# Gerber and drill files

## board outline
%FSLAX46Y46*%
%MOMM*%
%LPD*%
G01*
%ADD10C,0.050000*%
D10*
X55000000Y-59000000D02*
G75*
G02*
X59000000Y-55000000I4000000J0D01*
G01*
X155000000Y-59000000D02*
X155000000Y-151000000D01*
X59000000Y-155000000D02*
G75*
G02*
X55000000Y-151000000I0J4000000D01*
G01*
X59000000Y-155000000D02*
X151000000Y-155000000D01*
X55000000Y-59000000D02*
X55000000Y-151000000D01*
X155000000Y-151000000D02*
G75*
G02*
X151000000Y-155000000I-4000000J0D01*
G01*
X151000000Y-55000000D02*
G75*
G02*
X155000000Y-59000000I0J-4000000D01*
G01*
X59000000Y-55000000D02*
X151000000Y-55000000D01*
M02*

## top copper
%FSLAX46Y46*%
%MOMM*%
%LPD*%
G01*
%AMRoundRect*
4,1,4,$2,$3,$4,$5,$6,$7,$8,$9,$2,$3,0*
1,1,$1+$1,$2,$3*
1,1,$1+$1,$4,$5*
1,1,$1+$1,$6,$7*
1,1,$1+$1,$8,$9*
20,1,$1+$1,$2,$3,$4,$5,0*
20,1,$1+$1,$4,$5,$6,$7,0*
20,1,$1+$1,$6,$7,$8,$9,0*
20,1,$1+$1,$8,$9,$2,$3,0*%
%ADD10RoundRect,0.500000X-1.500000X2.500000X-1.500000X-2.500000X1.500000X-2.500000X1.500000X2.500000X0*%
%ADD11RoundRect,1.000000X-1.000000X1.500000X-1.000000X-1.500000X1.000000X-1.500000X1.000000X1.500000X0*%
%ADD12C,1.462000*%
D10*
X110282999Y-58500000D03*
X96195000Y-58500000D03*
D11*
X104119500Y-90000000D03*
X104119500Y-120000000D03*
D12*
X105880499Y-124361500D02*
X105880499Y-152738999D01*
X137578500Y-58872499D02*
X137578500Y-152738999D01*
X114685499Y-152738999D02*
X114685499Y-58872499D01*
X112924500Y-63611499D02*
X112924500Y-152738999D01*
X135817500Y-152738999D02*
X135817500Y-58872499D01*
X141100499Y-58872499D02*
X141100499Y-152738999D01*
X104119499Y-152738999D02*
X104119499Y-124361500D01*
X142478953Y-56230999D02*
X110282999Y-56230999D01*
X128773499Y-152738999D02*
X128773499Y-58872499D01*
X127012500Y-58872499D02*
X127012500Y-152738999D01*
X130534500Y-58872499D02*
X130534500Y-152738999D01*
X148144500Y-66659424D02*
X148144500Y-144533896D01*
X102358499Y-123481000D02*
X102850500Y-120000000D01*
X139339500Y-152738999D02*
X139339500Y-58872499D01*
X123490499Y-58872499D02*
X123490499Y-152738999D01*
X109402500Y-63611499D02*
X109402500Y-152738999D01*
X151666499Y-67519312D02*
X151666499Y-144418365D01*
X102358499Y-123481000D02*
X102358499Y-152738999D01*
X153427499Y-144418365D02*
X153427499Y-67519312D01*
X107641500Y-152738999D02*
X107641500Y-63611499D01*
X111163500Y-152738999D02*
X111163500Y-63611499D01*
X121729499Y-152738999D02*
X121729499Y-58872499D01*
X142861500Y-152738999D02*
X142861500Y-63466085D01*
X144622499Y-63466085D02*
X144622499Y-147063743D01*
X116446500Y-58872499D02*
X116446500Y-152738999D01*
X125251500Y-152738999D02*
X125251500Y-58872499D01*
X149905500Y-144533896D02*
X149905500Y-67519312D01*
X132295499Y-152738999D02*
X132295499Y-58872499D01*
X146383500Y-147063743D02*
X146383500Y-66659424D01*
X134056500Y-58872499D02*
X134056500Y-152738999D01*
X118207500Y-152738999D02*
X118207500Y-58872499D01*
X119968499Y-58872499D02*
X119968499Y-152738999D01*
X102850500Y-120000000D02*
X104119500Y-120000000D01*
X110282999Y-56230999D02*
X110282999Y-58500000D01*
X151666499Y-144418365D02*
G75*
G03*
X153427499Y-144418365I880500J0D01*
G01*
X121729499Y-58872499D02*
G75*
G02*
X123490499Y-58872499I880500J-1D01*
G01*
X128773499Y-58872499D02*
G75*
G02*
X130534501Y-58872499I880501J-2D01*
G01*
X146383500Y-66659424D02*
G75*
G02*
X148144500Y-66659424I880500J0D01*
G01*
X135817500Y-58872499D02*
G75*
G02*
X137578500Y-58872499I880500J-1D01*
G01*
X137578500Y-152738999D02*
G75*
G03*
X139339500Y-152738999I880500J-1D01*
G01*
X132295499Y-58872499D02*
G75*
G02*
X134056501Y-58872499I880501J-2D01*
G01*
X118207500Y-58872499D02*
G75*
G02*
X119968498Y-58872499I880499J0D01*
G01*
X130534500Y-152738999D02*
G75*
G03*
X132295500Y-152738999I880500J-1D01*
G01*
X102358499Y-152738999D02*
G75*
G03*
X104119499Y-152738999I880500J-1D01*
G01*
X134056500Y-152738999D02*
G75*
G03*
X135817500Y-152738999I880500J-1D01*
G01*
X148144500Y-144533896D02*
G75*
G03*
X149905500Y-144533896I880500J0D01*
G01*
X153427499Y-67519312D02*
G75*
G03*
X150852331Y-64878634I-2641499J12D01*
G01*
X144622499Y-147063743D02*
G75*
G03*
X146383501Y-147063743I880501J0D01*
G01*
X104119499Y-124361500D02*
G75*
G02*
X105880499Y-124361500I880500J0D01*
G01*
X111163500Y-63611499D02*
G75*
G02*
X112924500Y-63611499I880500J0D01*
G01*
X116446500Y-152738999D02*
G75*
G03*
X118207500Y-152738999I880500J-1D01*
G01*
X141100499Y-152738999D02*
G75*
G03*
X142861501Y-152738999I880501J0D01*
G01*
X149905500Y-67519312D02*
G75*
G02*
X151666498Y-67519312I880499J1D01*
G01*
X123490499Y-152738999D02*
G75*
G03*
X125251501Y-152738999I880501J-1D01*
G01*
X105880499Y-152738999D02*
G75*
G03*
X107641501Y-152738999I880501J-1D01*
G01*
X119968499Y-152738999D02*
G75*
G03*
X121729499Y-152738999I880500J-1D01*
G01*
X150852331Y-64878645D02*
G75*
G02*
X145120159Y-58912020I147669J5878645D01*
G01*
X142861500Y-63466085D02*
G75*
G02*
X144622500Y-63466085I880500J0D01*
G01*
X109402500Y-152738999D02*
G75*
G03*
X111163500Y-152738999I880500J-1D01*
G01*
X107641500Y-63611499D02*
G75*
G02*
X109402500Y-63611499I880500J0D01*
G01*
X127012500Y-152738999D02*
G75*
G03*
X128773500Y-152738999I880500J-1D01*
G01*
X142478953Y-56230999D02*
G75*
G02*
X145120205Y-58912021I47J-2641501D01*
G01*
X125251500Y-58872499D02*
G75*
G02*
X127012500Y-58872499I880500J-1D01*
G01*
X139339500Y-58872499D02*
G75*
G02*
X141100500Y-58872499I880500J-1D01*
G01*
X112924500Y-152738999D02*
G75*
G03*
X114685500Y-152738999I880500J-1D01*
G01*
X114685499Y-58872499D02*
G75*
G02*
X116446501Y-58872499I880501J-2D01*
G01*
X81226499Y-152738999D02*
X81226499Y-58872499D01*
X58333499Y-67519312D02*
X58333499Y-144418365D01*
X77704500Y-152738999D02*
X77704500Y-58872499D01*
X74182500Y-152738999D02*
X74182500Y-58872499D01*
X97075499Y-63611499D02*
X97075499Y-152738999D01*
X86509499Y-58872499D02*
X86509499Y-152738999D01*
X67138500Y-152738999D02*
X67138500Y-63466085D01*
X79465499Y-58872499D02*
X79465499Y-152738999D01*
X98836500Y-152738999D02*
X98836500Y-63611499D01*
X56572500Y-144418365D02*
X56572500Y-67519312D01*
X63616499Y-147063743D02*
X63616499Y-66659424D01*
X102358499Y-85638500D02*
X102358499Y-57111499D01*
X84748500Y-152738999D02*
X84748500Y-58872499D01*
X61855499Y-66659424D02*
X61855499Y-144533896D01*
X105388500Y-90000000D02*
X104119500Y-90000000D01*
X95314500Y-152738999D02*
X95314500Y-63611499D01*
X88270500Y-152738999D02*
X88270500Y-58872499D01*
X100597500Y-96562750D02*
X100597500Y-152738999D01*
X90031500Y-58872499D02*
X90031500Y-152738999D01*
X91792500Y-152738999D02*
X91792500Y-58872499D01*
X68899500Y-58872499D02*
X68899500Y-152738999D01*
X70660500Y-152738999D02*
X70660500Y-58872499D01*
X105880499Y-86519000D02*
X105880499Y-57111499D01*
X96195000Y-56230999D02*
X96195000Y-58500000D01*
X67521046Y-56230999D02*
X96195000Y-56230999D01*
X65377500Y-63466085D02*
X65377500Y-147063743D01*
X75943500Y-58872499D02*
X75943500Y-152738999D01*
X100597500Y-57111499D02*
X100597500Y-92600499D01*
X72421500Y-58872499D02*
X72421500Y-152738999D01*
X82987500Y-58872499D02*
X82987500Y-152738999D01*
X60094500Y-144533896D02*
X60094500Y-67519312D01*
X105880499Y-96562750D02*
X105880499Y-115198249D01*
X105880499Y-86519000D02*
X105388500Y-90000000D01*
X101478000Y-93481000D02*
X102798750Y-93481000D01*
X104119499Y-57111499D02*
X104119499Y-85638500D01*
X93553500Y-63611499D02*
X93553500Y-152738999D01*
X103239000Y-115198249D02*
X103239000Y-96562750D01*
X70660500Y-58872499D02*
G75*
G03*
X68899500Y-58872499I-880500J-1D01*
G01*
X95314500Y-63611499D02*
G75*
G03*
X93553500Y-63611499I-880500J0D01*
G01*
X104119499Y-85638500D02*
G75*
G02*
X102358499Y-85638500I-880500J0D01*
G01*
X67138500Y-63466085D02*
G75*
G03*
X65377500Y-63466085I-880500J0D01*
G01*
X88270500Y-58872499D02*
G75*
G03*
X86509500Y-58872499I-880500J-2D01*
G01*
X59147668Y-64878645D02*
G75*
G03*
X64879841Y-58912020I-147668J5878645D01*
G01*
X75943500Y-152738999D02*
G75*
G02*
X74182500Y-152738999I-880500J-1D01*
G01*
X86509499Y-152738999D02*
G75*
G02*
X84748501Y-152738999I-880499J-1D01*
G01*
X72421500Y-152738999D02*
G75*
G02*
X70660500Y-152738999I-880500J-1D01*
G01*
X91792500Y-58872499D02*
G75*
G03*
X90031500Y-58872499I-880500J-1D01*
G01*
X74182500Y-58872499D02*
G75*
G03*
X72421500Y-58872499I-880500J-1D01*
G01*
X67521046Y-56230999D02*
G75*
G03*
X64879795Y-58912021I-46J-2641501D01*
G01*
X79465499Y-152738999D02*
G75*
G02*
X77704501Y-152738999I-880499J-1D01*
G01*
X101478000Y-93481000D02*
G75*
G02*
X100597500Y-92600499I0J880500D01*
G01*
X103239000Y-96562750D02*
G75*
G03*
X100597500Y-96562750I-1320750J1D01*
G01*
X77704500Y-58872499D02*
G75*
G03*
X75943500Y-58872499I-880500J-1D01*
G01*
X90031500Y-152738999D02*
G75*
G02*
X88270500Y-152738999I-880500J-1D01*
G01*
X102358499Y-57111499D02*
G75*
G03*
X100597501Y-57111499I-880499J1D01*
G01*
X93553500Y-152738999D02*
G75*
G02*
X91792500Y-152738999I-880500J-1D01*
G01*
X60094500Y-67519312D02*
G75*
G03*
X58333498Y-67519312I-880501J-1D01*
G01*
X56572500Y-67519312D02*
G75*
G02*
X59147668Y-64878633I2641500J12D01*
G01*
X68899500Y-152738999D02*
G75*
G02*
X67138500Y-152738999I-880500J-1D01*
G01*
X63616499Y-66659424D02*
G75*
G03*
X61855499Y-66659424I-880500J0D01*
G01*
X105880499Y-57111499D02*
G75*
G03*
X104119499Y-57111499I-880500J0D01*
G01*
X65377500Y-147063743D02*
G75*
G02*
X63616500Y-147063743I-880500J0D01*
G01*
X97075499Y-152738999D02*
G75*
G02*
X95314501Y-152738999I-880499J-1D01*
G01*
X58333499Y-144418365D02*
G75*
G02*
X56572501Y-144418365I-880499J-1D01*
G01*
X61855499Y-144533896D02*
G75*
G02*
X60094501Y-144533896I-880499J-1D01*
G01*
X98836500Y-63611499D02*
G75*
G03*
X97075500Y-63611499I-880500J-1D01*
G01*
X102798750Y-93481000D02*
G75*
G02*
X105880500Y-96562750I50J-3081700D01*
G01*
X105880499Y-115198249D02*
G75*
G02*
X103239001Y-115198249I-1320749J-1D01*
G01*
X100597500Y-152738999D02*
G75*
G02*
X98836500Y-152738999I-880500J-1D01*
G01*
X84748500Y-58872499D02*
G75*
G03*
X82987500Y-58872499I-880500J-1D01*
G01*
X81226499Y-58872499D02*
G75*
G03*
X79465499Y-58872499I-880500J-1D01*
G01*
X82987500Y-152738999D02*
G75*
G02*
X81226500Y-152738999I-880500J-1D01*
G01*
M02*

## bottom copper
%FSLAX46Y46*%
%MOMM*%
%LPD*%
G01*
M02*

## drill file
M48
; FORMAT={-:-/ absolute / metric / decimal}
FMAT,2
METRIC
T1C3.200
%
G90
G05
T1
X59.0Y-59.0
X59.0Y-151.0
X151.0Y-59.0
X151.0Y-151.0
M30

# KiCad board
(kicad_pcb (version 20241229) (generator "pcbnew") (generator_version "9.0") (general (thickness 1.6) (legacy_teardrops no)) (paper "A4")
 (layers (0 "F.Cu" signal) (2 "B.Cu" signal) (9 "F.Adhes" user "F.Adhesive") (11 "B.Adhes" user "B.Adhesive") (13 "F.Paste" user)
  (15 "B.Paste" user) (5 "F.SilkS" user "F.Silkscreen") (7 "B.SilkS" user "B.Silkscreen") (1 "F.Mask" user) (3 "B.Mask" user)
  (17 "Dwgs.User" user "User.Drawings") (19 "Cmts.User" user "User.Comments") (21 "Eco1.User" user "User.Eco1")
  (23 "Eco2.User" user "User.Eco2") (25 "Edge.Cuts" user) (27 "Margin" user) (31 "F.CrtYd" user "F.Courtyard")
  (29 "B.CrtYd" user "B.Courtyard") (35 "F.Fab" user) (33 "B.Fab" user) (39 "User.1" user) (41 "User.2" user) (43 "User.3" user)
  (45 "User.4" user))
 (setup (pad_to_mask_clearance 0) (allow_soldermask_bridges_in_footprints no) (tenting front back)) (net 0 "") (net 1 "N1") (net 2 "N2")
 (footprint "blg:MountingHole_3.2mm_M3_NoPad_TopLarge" (layer "F.Cu") (at 151 59)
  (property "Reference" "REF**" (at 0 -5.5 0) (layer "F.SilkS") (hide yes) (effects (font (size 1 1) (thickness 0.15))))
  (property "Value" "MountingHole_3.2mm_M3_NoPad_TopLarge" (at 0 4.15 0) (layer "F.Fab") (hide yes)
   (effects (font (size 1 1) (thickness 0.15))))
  (pad "" np_thru_hole circle (at 0 0) (size 7.6 7.6) (drill 3.2) (layers) (zone_connect 2)))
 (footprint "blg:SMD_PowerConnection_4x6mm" (layer "F.Cu") (at 110.282999 58.5 -90)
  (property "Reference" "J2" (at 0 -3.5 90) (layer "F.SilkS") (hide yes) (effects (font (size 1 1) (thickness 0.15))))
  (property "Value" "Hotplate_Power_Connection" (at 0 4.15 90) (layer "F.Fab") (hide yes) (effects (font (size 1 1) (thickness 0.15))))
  (pad "1" smd roundrect (at 0 0 270) (size 6 4) (layers "F.Cu" "F.Mask" "F.Paste") (roundrect_rratio 0.125) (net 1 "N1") (zone_connect 2)))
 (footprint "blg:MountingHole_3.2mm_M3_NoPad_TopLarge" (layer "F.Cu") (at 59 151)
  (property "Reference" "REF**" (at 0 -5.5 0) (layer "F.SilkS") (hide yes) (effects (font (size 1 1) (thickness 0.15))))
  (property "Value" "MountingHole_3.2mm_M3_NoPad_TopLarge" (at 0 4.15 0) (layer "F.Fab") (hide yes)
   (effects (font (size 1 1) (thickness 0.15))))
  (pad "" np_thru_hole circle (at 0 0) (size 7.6 7.6) (drill 3.2) (layers) (zone_connect 2)))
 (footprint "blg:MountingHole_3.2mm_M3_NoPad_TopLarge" (layer "F.Cu") (at 151 151)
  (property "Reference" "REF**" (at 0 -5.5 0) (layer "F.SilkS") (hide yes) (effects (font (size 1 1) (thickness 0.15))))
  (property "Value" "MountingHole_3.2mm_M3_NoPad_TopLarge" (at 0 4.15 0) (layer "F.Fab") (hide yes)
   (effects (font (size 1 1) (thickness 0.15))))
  (pad "" np_thru_hole circle (at 0 0) (size 7.6 7.6) (drill 3.2) (layers) (zone_connect 2)))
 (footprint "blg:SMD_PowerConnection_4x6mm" (layer "F.Cu") (at 96.195 58.5 -90)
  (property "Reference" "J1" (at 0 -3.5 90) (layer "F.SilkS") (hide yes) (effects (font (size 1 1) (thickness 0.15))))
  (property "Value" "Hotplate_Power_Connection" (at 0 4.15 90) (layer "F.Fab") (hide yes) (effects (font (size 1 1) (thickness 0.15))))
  (pad "1" smd roundrect (at 0 0 270) (size 6 4) (layers "F.Cu" "F.Mask" "F.Paste") (roundrect_rratio 0.125) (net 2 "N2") (zone_connect 2)))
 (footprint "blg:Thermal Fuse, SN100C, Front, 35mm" (layer "F.Cu") (at 104.1195 105 -90)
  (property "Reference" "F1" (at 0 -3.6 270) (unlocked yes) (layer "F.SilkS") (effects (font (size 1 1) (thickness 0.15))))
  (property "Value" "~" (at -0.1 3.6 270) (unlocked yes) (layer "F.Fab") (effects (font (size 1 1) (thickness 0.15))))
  (pad "1" smd roundrect (at -15 0 270) (size 5 4) (layers "F.Cu" "F.Mask") (roundrect_rratio 0.25) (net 2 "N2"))
  (pad "2" smd roundrect (at 15 0 270) (size 5 4) (layers "F.Cu" "F.Mask") (roundrect_rratio 0.25) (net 1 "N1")))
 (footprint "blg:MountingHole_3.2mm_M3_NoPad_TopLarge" (layer "F.Cu") (at 59 59)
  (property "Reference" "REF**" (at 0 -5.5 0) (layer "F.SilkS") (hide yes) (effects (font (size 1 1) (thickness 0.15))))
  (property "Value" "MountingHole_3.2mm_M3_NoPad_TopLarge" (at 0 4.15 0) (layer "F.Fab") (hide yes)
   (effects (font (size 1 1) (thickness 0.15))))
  (pad "" np_thru_hole circle (at 0 0) (size 7.6 7.6) (drill 3.2) (layers) (zone_connect 2)))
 (gr_arc (start 55 59) (mid 56.171573 56.171573) (end 59 55) (stroke (width 0.05) (type solid)) (layer "Edge.Cuts"))
 (gr_line (start 155 59) (end 155 151) (stroke (width 0.05) (type default)) (layer "Edge.Cuts"))
 (gr_arc (start 59 155) (mid 56.171573 153.828427) (end 55 151) (stroke (width 0.05) (type solid)) (layer "Edge.Cuts"))
 (gr_line (start 59 155) (end 151 155) (stroke (width 0.05) (type default)) (layer "Edge.Cuts"))
 (gr_line (start 55 59) (end 55 151) (stroke (width 0.05) (type default)) (layer "Edge.Cuts"))
 (gr_arc (start 155 151) (mid 153.828427 153.828427) (end 151 155) (stroke (width 0.05) (type solid)) (layer "Edge.Cuts"))
 (gr_arc (start 151 55) (mid 153.828427 56.171573) (end 155 59) (stroke (width 0.05) (type solid)) (layer "Edge.Cuts"))
 (gr_line (start 59 55) (end 151 55) (stroke (width 0.05) (type default)) (layer "Edge.Cuts"))
 (segment (start 105.880499 124.3615) (end 105.880499 152.738999) (width 1.462) (layer "F.Cu") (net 1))
 (segment (start 137.5785 58.872499) (end 137.5785 152.738999) (width 1.462) (layer "F.Cu") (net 1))
 (segment (start 114.685499 152.738999) (end 114.685499 58.872499) (width 1.462) (layer "F.Cu") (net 1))
 (segment (start 112.9245 63.611499) (end 112.9245 152.738999) (width 1.462) (layer "F.Cu") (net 1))
 (segment (start 135.8175 152.738999) (end 135.8175 58.872499) (width 1.462) (layer "F.Cu") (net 1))
 (segment (start 141.100499 58.872499) (end 141.100499 152.738999) (width 1.462) (layer "F.Cu") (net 1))
 (segment (start 104.119499 152.738999) (end 104.119499 124.3615) (width 1.462) (layer "F.Cu") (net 1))
 (segment (start 142.478953 56.230999) (end 110.282999 56.230999) (width 1.462) (layer "F.Cu") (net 1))
 (segment (start 128.773499 152.738999) (end 128.773499 58.872499) (width 1.462) (layer "F.Cu") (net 1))
 (segment (start 127.0125 58.872499) (end 127.0125 152.738999) (width 1.462) (layer "F.Cu") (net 1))
 (segment (start 130.5345 58.872499) (end 130.5345 152.738999) (width 1.462) (layer "F.Cu") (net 1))
 (segment (start 148.1445 66.659424) (end 148.1445 144.533896) (width 1.462) (layer "F.Cu") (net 1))
 (segment (start 102.358499 123.481) (end 102.8505 120) (width 1.462) (layer "F.Cu") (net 1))
 (segment (start 139.3395 152.738999) (end 139.3395 58.872499) (width 1.462) (layer "F.Cu") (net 1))
 (segment (start 123.490499 58.872499) (end 123.490499 152.738999) (width 1.462) (layer "F.Cu") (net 1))
 (segment (start 109.4025 63.611499) (end 109.4025 152.738999) (width 1.462) (layer "F.Cu") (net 1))
 (segment (start 151.666499 67.519312) (end 151.666499 144.418365) (width 1.462) (layer "F.Cu") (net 1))
 (segment (start 102.358499 123.481) (end 102.358499 152.738999) (width 1.462) (layer "F.Cu") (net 1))
 (segment (start 153.427499 144.418365) (end 153.427499 67.519312) (width 1.462) (layer "F.Cu") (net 1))
 (segment (start 107.6415 152.738999) (end 107.6415 63.611499) (width 1.462) (layer "F.Cu") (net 1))
 (segment (start 111.1635 152.738999) (end 111.1635 63.611499) (width 1.462) (layer "F.Cu") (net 1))
 (segment (start 121.729499 152.738999) (end 121.729499 58.872499) (width 1.462) (layer "F.Cu") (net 1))
 (segment (start 142.8615 152.738999) (end 142.8615 63.466085) (width 1.462) (layer "F.Cu") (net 1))
 (segment (start 144.622499 63.466085) (end 144.622499 147.063743) (width 1.462) (layer "F.Cu") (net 1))
 (segment (start 116.4465 58.872499) (end 116.4465 152.738999) (width 1.462) (layer "F.Cu") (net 1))
 (segment (start 125.2515 152.738999) (end 125.2515 58.872499) (width 1.462) (layer "F.Cu") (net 1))
 (segment (start 149.9055 144.533896) (end 149.9055 67.519312) (width 1.462) (layer "F.Cu") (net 1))
 (segment (start 132.295499 152.738999) (end 132.295499 58.872499) (width 1.462) (layer "F.Cu") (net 1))
 (segment (start 146.3835 147.063743) (end 146.3835 66.659424) (width 1.462) (layer "F.Cu") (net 1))
 (segment (start 134.0565 58.872499) (end 134.0565 152.738999) (width 1.462) (layer "F.Cu") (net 1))
 (segment (start 118.2075 152.738999) (end 118.2075 58.872499) (width 1.462) (layer "F.Cu") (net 1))
 (segment (start 119.968499 58.872499) (end 119.968499 152.738999) (width 1.462) (layer "F.Cu") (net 1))
 (segment (start 102.8505 120) (end 104.1195 120) (width 1.462) (layer "F.Cu") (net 1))
 (segment (start 110.282999 56.230999) (end 110.282999 58.5) (width 1.462) (layer "F.Cu") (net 1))
 (arc (start 151.666499 144.418365) (mid 152.547 145.298865) (end 153.427499 144.418365) (width 1.462) (layer "F.Cu") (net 1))
 (arc (start 121.729499 58.872499) (mid 122.61 57.992) (end 123.490499 58.872499) (width 1.462) (layer "F.Cu") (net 1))
 (arc (start 128.773499 58.872499) (mid 129.654 57.992) (end 130.5345 58.872499) (width 1.462) (layer "F.Cu") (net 1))
 (arc (start 146.3835 66.659424) (mid 147.264 65.778924) (end 148.1445 66.659424) (width 1.462) (layer "F.Cu") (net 1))
 (arc (start 135.8175 58.872499) (mid 136.697999 57.992) (end 137.5785 58.872499) (width 1.462) (layer "F.Cu") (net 1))
 (arc (start 137.5785 152.738999) (mid 138.459 153.6195) (end 139.3395 152.738999) (width 1.462) (layer "F.Cu") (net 1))
 (arc (start 132.295499 58.872499) (mid 133.175999 57.992) (end 134.0565 58.872499) (width 1.462) (layer "F.Cu") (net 1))
 (arc (start 118.2075 58.872499) (mid 119.088 57.992) (end 119.968499 58.872499) (width 1.462) (layer "F.Cu") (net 1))
 (arc (start 130.5345 152.738999) (mid 131.414999 153.6195) (end 132.295499 152.738999) (width 1.462) (layer "F.Cu") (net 1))
 (arc (start 102.358499 152.738999) (mid 103.239 153.6195) (end 104.119499 152.738999) (width 1.462) (layer "F.Cu") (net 1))
 (arc (start 134.0565 152.738999) (mid 134.937 153.6195) (end 135.8175 152.738999) (width 1.462) (layer "F.Cu") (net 1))
 (arc (start 148.1445 144.533896) (mid 149.024999 145.414396) (end 149.9055 144.533896) (width 1.462) (layer "F.Cu") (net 1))
 (arc (start 153.427499 67.519312) (mid 152.683673 65.681825) (end 150.852331 64.878645) (width 1.462) (layer "F.Cu") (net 1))
 (arc (start 144.622499 147.063743) (mid 145.503 147.944243) (end 146.3835 147.063743) (width 1.462) (layer "F.Cu") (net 1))
 (arc (start 104.119499 124.3615) (mid 105 123.481) (end 105.880499 124.3615) (width 1.462) (layer "F.Cu") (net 1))
 (arc (start 111.1635 63.611499) (mid 112.044 62.730999) (end 112.9245 63.611499) (width 1.462) (layer "F.Cu") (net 1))
 (arc (start 116.4465 152.738999) (mid 117.327 153.6195) (end 118.2075 152.738999) (width 1.462) (layer "F.Cu") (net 1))
 (arc (start 141.100499 152.738999) (mid 141.981 153.6195) (end 142.8615 152.738999) (width 1.462) (layer "F.Cu") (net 1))
 (arc (start 149.9055 67.519312) (mid 150.786 66.638812) (end 151.666499 67.519312) (width 1.462) (layer "F.Cu") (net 1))
 (arc (start 123.490499 152.738999) (mid 124.371 153.6195) (end 125.2515 152.738999) (width 1.462) (layer "F.Cu") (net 1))
 (arc (start 105.880499 152.738999) (mid 106.761 153.6195) (end 107.6415 152.738999) (width 1.462) (layer "F.Cu") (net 1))
 (arc (start 119.968499 152.738999) (mid 120.849 153.6195) (end 121.729499 152.738999) (width 1.462) (layer "F.Cu") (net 1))
 (arc (start 150.852331 64.878645) (mid 146.759378 63.073991) (end 145.120158 58.91202) (width 1.462) (layer "F.Cu") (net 1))
 (arc (start 142.8615 63.466085) (mid 143.742 62.585585) (end 144.622499 63.466085) (width 1.462) (layer "F.Cu") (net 1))
 (arc (start 109.4025 152.738999) (mid 110.282999 153.6195) (end 111.1635 152.738999) (width 1.462) (layer "F.Cu") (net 1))
 (arc (start 107.6415 63.611499) (mid 108.521999 62.730999) (end 109.4025 63.611499) (width 1.462) (layer "F.Cu") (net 1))
 (arc (start 127.0125 152.738999) (mid 127.893 153.6195) (end 128.773499 152.738999) (width 1.462) (layer "F.Cu") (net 1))
 (arc (start 142.478953 56.230999) (mid 144.360697 57.018702) (end 145.120158 58.91202) (width 1.462) (layer "F.Cu") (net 1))
 (arc (start 125.2515 58.872499) (mid 126.131999 57.992) (end 127.0125 58.872499) (width 1.462) (layer "F.Cu") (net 1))
 (arc (start 139.3395 58.872499) (mid 140.219999 57.992) (end 141.100499 58.872499) (width 1.462) (layer "F.Cu") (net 1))
 (arc (start 112.9245 152.738999) (mid 113.805 153.6195) (end 114.685499 152.738999) (width 1.462) (layer "F.Cu") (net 1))
 (arc (start 114.685499 58.872499) (mid 115.565999 57.992) (end 116.4465 58.872499) (width 1.462) (layer "F.Cu") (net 1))
 (segment (start 81.226499 152.738999) (end 81.226499 58.872499) (width 1.462) (layer "F.Cu") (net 2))
 (segment (start 58.333499 67.519312) (end 58.333499 144.418365) (width 1.462) (layer "F.Cu") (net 2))
 (segment (start 77.7045 152.738999) (end 77.7045 58.872499) (width 1.462) (layer "F.Cu") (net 2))
 (segment (start 74.1825 152.738999) (end 74.1825 58.872499) (width 1.462) (layer "F.Cu") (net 2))
 (segment (start 97.075499 63.611499) (end 97.075499 152.738999) (width 1.462) (layer "F.Cu") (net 2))
 (segment (start 86.509499 58.872499) (end 86.509499 152.738999) (width 1.462) (layer "F.Cu") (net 2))
 (segment (start 67.1385 152.738999) (end 67.1385 63.466085) (width 1.462) (layer "F.Cu") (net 2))
 (segment (start 79.465499 58.872499) (end 79.465499 152.738999) (width 1.462) (layer "F.Cu") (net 2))
 (segment (start 98.8365 152.738999) (end 98.8365 63.611499) (width 1.462) (layer "F.Cu") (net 2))
 (segment (start 56.5725 144.418365) (end 56.5725 67.519312) (width 1.462) (layer "F.Cu") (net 2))
 (segment (start 63.616499 147.063743) (end 63.616499 66.659424) (width 1.462) (layer "F.Cu") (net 2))
 (segment (start 102.358499 85.6385) (end 102.358499 57.111499) (width 1.462) (layer "F.Cu") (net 2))
 (segment (start 84.7485 152.738999) (end 84.7485 58.872499) (width 1.462) (layer "F.Cu") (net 2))
 (segment (start 61.855499 66.659424) (end 61.855499 144.533896) (width 1.462) (layer "F.Cu") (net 2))
 (segment (start 105.3885 90) (end 104.1195 90) (width 1.462) (layer "F.Cu") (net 2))
 (segment (start 95.3145 152.738999) (end 95.3145 63.611499) (width 1.462) (layer "F.Cu") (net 2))
 (segment (start 88.2705 152.738999) (end 88.2705 58.872499) (width 1.462) (layer "F.Cu") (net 2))
 (segment (start 100.5975 96.56275) (end 100.5975 152.738999) (width 1.462) (layer "F.Cu") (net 2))
 (segment (start 90.0315 58.872499) (end 90.0315 152.738999) (width 1.462) (layer "F.Cu") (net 2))
 (segment (start 91.7925 152.738999) (end 91.7925 58.872499) (width 1.462) (layer "F.Cu") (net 2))
 (segment (start 68.8995 58.872499) (end 68.8995 152.738999) (width 1.462) (layer "F.Cu") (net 2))
 (segment (start 70.6605 152.738999) (end 70.6605 58.872499) (width 1.462) (layer "F.Cu") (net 2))
 (segment (start 105.880499 86.519) (end 105.880499 57.111499) (width 1.462) (layer "F.Cu") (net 2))
 (segment (start 96.195 56.230999) (end 96.195 58.5) (width 1.462) (layer "F.Cu") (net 2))
 (segment (start 67.521046 56.230999) (end 96.195 56.230999) (width 1.462) (layer "F.Cu") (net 2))
 (segment (start 65.3775 63.466085) (end 65.3775 147.063743) (width 1.462) (layer "F.Cu") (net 2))
 (segment (start 75.9435 58.872499) (end 75.9435 152.738999) (width 1.462) (layer "F.Cu") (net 2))
 (segment (start 100.5975 57.111499) (end 100.5975 92.600499) (width 1.462) (layer "F.Cu") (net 2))
 (segment (start 72.4215 58.872499) (end 72.4215 152.738999) (width 1.462) (layer "F.Cu") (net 2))
 (segment (start 82.9875 58.872499) (end 82.9875 152.738999) (width 1.462) (layer "F.Cu") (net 2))
 (segment (start 60.0945 144.533896) (end 60.0945 67.519312) (width 1.462) (layer "F.Cu") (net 2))
 (segment (start 105.880499 96.56275) (end 105.880499 115.198249) (width 1.462) (layer "F.Cu") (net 2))
 (segment (start 105.880499 86.519) (end 105.3885 90) (width 1.462) (layer "F.Cu") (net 2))
 (segment (start 101.478 93.481) (end 102.79875 93.481) (width 1.462) (layer "F.Cu") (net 2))
 (segment (start 104.119499 57.111499) (end 104.119499 85.6385) (width 1.462) (layer "F.Cu") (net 2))
 (segment (start 93.5535 63.611499) (end 93.5535 152.738999) (width 1.462) (layer "F.Cu") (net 2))
 (segment (start 103.239 115.198249) (end 103.239 96.56275) (width 1.462) (layer "F.Cu") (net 2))
 (arc (start 70.6605 58.872499) (mid 69.78 57.992) (end 68.8995 58.872499) (width 1.462) (layer "F.Cu") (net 2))
 (arc (start 95.3145 63.611499) (mid 94.433999 62.730999) (end 93.5535 63.611499) (width 1.462) (layer "F.Cu") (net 2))
 (arc (start 104.119499 85.6385) (mid 103.239 86.519) (end 102.358499 85.6385) (width 1.462) (layer "F.Cu") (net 2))
 (arc (start 67.1385 63.466085) (mid 66.257999 62.585585) (end 65.3775 63.466085) (width 1.462) (layer "F.Cu") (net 2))
 (arc (start 88.2705 58.872499) (mid 87.39 57.992) (end 86.509499 58.872499) (width 1.462) (layer "F.Cu") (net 2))
 (arc (start 59.147668 64.878645) (mid 63.240621 63.073991) (end 64.879841 58.91202) (width 1.462) (layer "F.Cu") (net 2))
 (arc (start 75.9435 152.738999) (mid 75.062999 153.6195) (end 74.1825 152.738999) (width 1.462) (layer "F.Cu") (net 2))
 (arc (start 86.509499 152.738999) (mid 85.628999 153.6195) (end 84.7485 152.738999) (width 1.462) (layer "F.Cu") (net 2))
 (arc (start 72.4215 152.738999) (mid 71.541 153.6195) (end 70.6605 152.738999) (width 1.462) (layer "F.Cu") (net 2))
 (arc (start 91.7925 58.872499) (mid 90.911999 57.992) (end 90.0315 58.872499) (width 1.462) (layer "F.Cu") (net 2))
 (arc (start 74.1825 58.872499) (mid 73.301999 57.992) (end 72.4215 58.872499) (width 1.462) (layer "F.Cu") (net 2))
 (arc (start 67.521046 56.230999) (mid 65.639302 57.018702) (end 64.879841 58.91202) (width 1.462) (layer "F.Cu") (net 2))
 (arc (start 79.465499 152.738999) (mid 78.585 153.6195) (end 77.7045 152.738999) (width 1.462) (layer "F.Cu") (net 2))
 (arc (start 101.478 93.481) (mid 100.855392 93.223107) (end 100.5975 92.600499) (width 1.462) (layer "F.Cu") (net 2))
 (arc (start 103.239 96.56275) (mid 101.91825 95.241999) (end 100.5975 96.56275) (width 1.462) (layer "F.Cu") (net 2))
 (arc (start 77.7045 58.872499) (mid 76.824 57.992) (end 75.9435 58.872499) (width 1.462) (layer "F.Cu") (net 2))
 (arc (start 90.0315 152.738999) (mid 89.151 153.6195) (end 88.2705 152.738999) (width 1.462) (layer "F.Cu") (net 2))
 (arc (start 102.358499 57.111499) (mid 101.477999 56.230999) (end 100.5975 57.111499) (width 1.462) (layer "F.Cu") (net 2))
 (arc (start 93.5535 152.738999) (mid 92.672999 153.6195) (end 91.7925 152.738999) (width 1.462) (layer "F.Cu") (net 2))
 (arc (start 60.0945 67.519312) (mid 59.214 66.638812) (end 58.333499 67.519312) (width 1.462) (layer "F.Cu") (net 2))
 (arc (start 56.5725 67.519312) (mid 57.316326 65.681825) (end 59.147668 64.878645) (width 1.462) (layer "F.Cu") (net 2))
 (arc (start 68.8995 152.738999) (mid 68.018999 153.6195) (end 67.1385 152.738999) (width 1.462) (layer "F.Cu") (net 2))
 (arc (start 63.616499 66.659424) (mid 62.736 65.778924) (end 61.855499 66.659424) (width 1.462) (layer "F.Cu") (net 2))
 (arc (start 105.880499 57.111499) (mid 105 56.230999) (end 104.119499 57.111499) (width 1.462) (layer "F.Cu") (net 2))
 (arc (start 65.3775 147.063743) (mid 64.497 147.944243) (end 63.616499 147.063743) (width 1.462) (layer "F.Cu") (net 2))
 (arc (start 97.075499 152.738999) (mid 96.195 153.6195) (end 95.3145 152.738999) (width 1.462) (layer "F.Cu") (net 2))
 (arc (start 58.333499 144.418365) (mid 57.452999 145.298865) (end 56.5725 144.418365) (width 1.462) (layer "F.Cu") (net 2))
 (arc (start 61.855499 144.533896) (mid 60.974999 145.414396) (end 60.0945 144.533896) (width 1.462) (layer "F.Cu") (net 2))
 (arc (start 98.8365 63.611499) (mid 97.956 62.730999) (end 97.075499 63.611499) (width 1.462) (layer "F.Cu") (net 2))
 (arc (start 102.79875 93.481) (mid 104.977876 94.383623) (end 105.880499 96.56275) (width 1.462) (layer "F.Cu") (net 2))
 (arc (start 105.880499 115.198249) (mid 104.55975 116.518999) (end 103.239 115.198249) (width 1.462) (layer "F.Cu") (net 2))
 (arc (start 100.5975 152.738999) (mid 99.717 153.6195) (end 98.8365 152.738999) (width 1.462) (layer "F.Cu") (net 2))
 (arc (start 84.7485 58.872499) (mid 83.868 57.992) (end 82.9875 58.872499) (width 1.462) (layer "F.Cu") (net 2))
 (arc (start 81.226499 58.872499) (mid 80.346 57.992) (end 79.465499 58.872499) (width 1.462) (layer "F.Cu") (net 2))
 (arc (start 82.9875 152.738999) (mid 82.107 153.6195) (end 81.226499 152.738999) (width 1.462) (layer "F.Cu") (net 2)))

